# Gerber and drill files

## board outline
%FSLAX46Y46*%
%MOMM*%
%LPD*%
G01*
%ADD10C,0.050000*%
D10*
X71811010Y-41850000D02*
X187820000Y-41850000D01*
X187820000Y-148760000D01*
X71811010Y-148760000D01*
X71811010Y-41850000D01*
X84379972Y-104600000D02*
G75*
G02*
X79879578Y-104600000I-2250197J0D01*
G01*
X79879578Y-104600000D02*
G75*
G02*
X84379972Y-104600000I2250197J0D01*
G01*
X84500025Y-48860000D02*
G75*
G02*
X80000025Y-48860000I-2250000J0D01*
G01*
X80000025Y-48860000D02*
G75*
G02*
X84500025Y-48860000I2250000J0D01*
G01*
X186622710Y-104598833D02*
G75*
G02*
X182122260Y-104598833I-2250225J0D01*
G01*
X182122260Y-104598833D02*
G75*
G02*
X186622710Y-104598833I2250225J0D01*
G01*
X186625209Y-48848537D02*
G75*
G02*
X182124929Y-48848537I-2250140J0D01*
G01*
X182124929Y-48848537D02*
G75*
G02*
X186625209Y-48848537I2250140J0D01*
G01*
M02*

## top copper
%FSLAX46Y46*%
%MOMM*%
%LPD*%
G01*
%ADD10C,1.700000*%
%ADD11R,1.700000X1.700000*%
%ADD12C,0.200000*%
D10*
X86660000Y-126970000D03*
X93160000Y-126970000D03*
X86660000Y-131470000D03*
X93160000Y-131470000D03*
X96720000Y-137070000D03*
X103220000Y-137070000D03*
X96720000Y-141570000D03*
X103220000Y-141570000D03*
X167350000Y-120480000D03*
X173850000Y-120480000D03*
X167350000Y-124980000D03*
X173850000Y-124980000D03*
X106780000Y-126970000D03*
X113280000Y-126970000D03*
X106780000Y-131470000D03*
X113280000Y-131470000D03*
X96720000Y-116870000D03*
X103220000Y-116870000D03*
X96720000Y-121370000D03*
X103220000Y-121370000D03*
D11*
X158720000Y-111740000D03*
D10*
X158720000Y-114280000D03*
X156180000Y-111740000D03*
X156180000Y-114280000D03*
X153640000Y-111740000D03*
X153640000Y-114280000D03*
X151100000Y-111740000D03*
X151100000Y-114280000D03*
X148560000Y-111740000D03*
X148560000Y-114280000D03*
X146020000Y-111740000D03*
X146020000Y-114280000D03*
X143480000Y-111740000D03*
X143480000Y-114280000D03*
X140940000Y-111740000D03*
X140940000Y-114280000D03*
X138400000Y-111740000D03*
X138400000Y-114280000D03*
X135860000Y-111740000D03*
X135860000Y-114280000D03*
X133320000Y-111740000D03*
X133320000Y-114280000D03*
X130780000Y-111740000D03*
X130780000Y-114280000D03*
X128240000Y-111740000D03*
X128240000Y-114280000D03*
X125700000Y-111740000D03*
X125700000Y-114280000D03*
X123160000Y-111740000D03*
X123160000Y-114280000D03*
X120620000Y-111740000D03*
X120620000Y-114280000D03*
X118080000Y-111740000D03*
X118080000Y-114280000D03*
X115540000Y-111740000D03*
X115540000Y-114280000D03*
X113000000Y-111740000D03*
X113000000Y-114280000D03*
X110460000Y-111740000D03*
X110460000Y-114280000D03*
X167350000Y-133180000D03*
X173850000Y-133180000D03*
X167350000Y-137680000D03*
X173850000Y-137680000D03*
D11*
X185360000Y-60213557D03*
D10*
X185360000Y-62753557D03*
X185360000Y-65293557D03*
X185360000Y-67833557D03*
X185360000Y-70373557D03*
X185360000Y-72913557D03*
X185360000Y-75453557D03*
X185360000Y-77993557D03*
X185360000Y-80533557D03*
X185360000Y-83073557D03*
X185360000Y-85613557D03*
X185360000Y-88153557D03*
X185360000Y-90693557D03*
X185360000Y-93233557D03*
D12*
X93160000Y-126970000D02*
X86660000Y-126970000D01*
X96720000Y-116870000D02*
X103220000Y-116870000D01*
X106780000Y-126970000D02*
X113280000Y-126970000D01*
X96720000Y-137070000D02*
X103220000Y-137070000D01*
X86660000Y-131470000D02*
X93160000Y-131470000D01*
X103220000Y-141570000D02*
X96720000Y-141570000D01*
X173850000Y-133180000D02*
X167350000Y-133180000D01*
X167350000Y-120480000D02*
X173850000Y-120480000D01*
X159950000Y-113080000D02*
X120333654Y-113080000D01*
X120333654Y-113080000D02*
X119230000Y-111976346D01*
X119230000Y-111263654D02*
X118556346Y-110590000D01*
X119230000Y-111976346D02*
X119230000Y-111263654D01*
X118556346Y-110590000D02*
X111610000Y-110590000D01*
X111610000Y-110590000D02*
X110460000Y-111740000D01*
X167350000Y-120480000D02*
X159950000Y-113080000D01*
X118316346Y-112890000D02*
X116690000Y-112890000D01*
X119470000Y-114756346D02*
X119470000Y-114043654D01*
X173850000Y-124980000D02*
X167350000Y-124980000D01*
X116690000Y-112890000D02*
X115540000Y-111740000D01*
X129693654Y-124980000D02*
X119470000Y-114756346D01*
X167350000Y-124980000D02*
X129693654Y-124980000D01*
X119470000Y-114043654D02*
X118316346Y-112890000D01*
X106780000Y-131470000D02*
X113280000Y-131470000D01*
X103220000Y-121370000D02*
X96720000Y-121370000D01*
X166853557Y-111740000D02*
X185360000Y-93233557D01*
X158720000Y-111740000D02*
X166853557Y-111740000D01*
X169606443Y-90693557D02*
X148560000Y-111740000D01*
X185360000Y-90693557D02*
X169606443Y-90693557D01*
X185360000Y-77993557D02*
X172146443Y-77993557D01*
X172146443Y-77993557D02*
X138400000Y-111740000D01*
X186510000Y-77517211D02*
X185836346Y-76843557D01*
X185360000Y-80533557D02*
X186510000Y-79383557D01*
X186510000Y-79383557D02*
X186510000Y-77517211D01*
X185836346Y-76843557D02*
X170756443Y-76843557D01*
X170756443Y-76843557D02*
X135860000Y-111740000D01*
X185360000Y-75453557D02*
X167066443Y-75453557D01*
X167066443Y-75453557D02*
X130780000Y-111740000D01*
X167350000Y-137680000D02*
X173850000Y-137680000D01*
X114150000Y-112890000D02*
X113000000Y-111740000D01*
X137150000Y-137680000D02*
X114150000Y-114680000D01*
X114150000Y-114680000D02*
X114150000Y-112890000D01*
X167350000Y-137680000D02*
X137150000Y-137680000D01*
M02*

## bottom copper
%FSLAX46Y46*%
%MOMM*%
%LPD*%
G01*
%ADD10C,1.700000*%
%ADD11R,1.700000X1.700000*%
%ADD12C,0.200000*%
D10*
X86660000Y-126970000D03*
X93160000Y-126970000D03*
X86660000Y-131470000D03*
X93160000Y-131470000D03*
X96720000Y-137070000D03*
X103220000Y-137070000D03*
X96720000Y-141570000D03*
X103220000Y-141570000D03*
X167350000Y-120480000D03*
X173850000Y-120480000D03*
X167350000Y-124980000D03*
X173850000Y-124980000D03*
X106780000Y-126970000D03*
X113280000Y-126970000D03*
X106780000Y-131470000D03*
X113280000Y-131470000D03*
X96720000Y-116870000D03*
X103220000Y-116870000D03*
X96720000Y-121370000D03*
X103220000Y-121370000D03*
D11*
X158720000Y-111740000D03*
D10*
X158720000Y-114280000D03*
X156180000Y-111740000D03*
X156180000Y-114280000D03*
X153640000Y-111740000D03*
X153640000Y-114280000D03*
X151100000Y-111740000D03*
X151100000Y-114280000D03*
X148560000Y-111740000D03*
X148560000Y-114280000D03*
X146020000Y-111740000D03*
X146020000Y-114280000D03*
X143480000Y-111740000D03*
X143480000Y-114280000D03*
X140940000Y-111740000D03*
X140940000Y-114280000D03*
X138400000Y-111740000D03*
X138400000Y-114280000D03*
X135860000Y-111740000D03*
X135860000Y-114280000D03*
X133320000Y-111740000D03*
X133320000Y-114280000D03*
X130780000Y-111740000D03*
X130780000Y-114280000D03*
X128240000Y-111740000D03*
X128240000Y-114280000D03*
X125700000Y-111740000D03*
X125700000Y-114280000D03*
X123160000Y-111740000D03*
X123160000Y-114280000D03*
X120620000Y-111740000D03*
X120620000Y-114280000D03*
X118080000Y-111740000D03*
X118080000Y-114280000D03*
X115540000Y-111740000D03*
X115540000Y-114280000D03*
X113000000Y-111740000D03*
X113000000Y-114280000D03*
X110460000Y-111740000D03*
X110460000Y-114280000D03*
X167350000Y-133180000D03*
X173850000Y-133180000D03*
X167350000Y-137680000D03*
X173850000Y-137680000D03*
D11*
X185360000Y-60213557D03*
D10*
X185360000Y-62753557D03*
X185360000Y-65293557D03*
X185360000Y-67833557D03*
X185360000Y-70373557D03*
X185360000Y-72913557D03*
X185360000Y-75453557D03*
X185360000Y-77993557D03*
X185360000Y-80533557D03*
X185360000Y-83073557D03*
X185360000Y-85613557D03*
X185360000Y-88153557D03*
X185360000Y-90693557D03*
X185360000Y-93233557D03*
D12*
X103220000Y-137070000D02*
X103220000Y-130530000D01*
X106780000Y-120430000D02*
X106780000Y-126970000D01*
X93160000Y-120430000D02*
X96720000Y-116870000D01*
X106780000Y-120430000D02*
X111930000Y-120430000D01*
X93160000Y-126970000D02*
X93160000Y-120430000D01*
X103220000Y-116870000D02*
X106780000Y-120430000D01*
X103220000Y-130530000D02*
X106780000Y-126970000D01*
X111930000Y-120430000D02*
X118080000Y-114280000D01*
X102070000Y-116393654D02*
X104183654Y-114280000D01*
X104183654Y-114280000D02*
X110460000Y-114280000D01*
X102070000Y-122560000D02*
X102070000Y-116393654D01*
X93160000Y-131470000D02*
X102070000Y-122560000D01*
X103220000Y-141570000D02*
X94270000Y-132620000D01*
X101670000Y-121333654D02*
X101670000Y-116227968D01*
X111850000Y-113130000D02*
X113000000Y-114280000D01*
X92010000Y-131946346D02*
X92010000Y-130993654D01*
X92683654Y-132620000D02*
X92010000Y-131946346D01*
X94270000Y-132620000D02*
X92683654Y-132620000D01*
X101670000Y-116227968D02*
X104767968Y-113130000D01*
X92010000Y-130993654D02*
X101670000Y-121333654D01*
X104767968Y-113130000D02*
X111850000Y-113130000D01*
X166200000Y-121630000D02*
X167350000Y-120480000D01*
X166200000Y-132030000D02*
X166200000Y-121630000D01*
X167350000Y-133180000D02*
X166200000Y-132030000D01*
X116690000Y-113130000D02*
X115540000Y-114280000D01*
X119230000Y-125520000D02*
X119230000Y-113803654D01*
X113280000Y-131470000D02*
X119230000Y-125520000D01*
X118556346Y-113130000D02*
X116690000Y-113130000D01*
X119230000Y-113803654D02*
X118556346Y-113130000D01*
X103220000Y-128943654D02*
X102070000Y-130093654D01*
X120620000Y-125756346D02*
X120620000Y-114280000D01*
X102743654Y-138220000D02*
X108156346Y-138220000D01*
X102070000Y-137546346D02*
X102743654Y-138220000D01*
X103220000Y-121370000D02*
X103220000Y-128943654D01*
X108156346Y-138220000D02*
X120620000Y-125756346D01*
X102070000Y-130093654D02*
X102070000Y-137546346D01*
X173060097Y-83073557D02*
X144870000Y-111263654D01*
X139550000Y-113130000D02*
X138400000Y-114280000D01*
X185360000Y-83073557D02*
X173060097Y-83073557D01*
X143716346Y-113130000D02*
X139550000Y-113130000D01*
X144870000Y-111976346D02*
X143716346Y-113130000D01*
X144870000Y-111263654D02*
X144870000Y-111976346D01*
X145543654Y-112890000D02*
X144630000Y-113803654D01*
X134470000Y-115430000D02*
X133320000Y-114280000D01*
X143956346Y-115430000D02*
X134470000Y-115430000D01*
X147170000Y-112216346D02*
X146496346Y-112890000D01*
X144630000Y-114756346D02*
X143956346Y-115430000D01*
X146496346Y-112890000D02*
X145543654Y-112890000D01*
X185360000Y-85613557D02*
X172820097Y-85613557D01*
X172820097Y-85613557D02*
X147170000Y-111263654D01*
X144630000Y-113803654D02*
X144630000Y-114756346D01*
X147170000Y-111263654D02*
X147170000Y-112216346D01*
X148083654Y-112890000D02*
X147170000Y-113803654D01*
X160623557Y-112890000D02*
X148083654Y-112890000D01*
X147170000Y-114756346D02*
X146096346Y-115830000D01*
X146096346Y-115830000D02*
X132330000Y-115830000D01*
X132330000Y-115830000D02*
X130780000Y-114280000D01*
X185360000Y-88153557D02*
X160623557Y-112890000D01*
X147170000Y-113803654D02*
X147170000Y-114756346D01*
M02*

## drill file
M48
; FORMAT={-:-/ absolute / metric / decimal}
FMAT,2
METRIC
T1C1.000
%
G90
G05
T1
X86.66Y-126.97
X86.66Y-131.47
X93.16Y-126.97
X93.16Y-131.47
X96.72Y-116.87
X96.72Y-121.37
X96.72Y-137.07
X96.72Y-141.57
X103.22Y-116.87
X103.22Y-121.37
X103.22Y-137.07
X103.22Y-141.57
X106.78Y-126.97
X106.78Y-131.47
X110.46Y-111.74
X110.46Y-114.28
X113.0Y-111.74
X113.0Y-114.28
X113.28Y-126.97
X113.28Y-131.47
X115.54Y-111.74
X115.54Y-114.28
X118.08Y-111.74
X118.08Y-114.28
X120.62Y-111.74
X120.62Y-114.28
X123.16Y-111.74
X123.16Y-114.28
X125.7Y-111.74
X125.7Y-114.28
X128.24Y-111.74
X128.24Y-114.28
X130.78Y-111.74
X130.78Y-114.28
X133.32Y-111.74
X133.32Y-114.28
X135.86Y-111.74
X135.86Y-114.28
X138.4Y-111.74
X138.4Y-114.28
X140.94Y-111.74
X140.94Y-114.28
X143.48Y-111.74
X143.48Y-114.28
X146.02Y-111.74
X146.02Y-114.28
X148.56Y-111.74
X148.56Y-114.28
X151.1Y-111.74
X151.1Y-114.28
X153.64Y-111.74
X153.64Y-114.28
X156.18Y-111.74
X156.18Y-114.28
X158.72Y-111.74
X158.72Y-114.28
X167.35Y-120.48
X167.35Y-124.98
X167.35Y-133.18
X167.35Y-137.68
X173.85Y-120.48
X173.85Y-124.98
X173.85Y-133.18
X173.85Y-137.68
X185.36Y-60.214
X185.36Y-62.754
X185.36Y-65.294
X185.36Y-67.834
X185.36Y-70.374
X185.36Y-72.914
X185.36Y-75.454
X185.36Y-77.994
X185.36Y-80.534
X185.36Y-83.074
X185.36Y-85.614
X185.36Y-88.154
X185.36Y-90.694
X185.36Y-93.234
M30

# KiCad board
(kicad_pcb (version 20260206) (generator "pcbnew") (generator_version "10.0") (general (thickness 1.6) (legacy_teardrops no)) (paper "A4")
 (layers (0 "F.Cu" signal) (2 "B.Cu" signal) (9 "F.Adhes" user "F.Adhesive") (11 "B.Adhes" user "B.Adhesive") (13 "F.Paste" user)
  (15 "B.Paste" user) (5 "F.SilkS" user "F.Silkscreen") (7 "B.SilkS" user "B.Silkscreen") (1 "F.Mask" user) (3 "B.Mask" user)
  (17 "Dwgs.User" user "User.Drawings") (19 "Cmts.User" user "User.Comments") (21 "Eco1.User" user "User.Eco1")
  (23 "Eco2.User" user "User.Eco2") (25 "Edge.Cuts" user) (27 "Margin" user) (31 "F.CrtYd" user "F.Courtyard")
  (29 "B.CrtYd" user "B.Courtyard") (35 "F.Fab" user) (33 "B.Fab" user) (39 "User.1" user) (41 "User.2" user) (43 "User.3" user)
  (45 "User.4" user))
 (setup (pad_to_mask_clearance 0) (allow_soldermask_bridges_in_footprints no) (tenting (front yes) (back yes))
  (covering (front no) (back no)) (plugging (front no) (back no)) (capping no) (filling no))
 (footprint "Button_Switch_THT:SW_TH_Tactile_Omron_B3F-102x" (layer "F.Cu") (at 86.66 126.97)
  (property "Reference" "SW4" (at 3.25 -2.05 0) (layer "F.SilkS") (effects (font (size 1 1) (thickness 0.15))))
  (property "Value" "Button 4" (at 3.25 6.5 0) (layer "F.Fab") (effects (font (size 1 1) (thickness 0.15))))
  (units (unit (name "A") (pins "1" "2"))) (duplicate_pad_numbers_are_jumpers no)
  (pad "1" thru_hole circle (at 0 0) (size 1.7 1.7) (drill 1) (layers "*.Cu" "*.Mask") (remove_unused_layers no) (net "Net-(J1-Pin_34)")
   (thermal_bridge_angle 90))
  (pad "1" thru_hole circle (at 6.5 0) (size 1.7 1.7) (drill 1) (layers "*.Cu" "*.Mask") (remove_unused_layers no) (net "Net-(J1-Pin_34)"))
  (pad "2" thru_hole circle (at 0 4.5) (size 1.7 1.7) (drill 1) (layers "*.Cu" "*.Mask") (remove_unused_layers no) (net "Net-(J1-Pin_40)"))
  (pad "2" thru_hole circle (at 6.5 4.5) (size 1.7 1.7) (drill 1) (layers "*.Cu" "*.Mask") (remove_unused_layers no) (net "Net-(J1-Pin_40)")))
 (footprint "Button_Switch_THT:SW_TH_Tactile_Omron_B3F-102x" (layer "F.Cu") (at 96.72 137.07)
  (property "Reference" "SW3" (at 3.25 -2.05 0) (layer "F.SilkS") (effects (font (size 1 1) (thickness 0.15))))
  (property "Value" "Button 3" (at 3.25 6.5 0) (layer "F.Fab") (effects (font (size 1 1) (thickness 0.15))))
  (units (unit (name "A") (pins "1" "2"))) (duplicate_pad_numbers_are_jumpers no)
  (pad "1" thru_hole circle (at 0 0) (size 1.7 1.7) (drill 1) (layers "*.Cu" "*.Mask") (remove_unused_layers no) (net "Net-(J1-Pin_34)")
   (thermal_bridge_angle 90))
  (pad "1" thru_hole circle (at 6.5 0) (size 1.7 1.7) (drill 1) (layers "*.Cu" "*.Mask") (remove_unused_layers no) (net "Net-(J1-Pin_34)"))
  (pad "2" thru_hole circle (at 0 4.5) (size 1.7 1.7) (drill 1) (layers "*.Cu" "*.Mask") (remove_unused_layers no) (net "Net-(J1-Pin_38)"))
  (pad "2" thru_hole circle (at 6.5 4.5) (size 1.7 1.7) (drill 1) (layers "*.Cu" "*.Mask") (remove_unused_layers no) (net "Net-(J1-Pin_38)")))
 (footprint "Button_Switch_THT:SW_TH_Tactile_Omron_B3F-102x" (layer "F.Cu") (at 167.35 120.48)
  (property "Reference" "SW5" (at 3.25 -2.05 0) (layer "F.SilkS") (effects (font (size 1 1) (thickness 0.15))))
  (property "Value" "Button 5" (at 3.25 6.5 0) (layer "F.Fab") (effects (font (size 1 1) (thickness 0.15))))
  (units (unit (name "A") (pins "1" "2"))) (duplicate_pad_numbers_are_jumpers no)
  (pad "1" thru_hole circle (at 0 0) (size 1.7 1.7) (drill 1) (layers "*.Cu" "*.Mask") (remove_unused_layers no) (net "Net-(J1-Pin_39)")
   (thermal_bridge_angle 90))
  (pad "1" thru_hole circle (at 6.5 0) (size 1.7 1.7) (drill 1) (layers "*.Cu" "*.Mask") (remove_unused_layers no) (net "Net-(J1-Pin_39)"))
  (pad "2" thru_hole circle (at 0 4.5) (size 1.7 1.7) (drill 1) (layers "*.Cu" "*.Mask") (remove_unused_layers no) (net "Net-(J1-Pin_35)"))
  (pad "2" thru_hole circle (at 6.5 4.5) (size 1.7 1.7) (drill 1) (layers "*.Cu" "*.Mask") (remove_unused_layers no) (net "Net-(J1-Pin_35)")))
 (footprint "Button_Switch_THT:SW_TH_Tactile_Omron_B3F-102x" (layer "F.Cu") (at 106.78 126.97)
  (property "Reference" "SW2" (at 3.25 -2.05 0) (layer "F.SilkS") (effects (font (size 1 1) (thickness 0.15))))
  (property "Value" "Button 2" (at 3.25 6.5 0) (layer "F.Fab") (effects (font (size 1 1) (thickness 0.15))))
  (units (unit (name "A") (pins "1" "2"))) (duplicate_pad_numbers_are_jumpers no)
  (pad "1" thru_hole circle (at 0 0) (size 1.7 1.7) (drill 1) (layers "*.Cu" "*.Mask") (remove_unused_layers no) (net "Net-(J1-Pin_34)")
   (thermal_bridge_angle 90))
  (pad "1" thru_hole circle (at 6.5 0) (size 1.7 1.7) (drill 1) (layers "*.Cu" "*.Mask") (remove_unused_layers no) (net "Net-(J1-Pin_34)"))
  (pad "2" thru_hole circle (at 0 4.5) (size 1.7 1.7) (drill 1) (layers "*.Cu" "*.Mask") (remove_unused_layers no) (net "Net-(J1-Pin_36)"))
  (pad "2" thru_hole circle (at 6.5 4.5) (size 1.7 1.7) (drill 1) (layers "*.Cu" "*.Mask") (remove_unused_layers no) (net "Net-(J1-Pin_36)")))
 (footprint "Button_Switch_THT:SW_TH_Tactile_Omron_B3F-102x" (layer "F.Cu") (at 96.72 116.87)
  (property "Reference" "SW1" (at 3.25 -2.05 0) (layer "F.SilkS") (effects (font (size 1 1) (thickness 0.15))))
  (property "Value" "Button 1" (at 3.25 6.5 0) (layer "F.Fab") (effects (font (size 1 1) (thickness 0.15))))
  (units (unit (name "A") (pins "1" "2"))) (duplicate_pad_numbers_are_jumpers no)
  (pad "1" thru_hole circle (at 0 0) (size 1.7 1.7) (drill 1) (layers "*.Cu" "*.Mask") (remove_unused_layers no) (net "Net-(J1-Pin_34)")
   (thermal_bridge_angle 90))
  (pad "1" thru_hole circle (at 6.5 0) (size 1.7 1.7) (drill 1) (layers "*.Cu" "*.Mask") (remove_unused_layers no) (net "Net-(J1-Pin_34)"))
  (pad "2" thru_hole circle (at 0 4.5) (size 1.7 1.7) (drill 1) (layers "*.Cu" "*.Mask") (remove_unused_layers no) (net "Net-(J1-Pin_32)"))
  (pad "2" thru_hole circle (at 6.5 4.5) (size 1.7 1.7) (drill 1) (layers "*.Cu" "*.Mask") (remove_unused_layers no) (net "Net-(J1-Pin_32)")))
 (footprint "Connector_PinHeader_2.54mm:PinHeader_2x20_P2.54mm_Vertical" (layer "F.Cu") (at 158.72 111.74 -90)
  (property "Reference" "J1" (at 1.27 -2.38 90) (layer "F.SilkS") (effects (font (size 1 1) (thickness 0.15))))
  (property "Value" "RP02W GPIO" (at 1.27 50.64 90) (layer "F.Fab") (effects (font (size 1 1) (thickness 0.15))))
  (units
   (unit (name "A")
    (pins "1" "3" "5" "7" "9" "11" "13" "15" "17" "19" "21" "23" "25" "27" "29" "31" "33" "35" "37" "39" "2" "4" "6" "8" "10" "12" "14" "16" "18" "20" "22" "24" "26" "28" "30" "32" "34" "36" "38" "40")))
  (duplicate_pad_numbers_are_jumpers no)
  (pad "1" thru_hole rect (at 0 0 270) (size 1.7 1.7) (drill 1) (layers "*.Cu" "*.Mask") (remove_unused_layers no) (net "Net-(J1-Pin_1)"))
  (pad "2" thru_hole circle (at 2.54 0 270) (size 1.7 1.7) (drill 1) (layers "*.Cu" "*.Mask") (remove_unused_layers no)
   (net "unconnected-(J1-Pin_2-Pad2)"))
  (pad "3" thru_hole circle (at 0 2.54 270) (size 1.7 1.7) (drill 1) (layers "*.Cu" "*.Mask") (remove_unused_layers no)
   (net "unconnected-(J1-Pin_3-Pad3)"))
  (pad "4" thru_hole circle (at 2.54 2.54 270) (size 1.7 1.7) (drill 1) (layers "*.Cu" "*.Mask") (remove_unused_layers no)
   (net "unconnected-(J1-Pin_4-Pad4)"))
  (pad "5" thru_hole circle (at 0 5.08 270) (size 1.7 1.7) (drill 1) (layers "*.Cu" "*.Mask") (remove_unused_layers no)
   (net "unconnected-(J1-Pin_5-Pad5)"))
  (pad "6" thru_hole circle (at 2.54 5.08 270) (size 1.7 1.7) (drill 1) (layers "*.Cu" "*.Mask") (remove_unused_layers no)
   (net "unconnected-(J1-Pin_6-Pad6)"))
  (pad "7" thru_hole circle (at 0 7.62 270) (size 1.7 1.7) (drill 1) (layers "*.Cu" "*.Mask") (remove_unused_layers no)
   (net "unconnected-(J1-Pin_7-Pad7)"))
  (pad "8" thru_hole circle (at 2.54 7.62 270) (size 1.7 1.7) (drill 1) (layers "*.Cu" "*.Mask") (remove_unused_layers no)
   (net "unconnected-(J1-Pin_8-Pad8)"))
  (pad "9" thru_hole circle (at 0 10.16 270) (size 1.7 1.7) (drill 1) (layers "*.Cu" "*.Mask") (remove_unused_layers no)
   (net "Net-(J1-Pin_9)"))
  (pad "10" thru_hole circle (at 2.54 10.16 270) (size 1.7 1.7) (drill 1) (layers "*.Cu" "*.Mask") (remove_unused_layers no)
   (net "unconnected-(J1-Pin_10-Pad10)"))
  (pad "11" thru_hole circle (at 0 12.7 270) (size 1.7 1.7) (drill 1) (layers "*.Cu" "*.Mask") (remove_unused_layers no)
   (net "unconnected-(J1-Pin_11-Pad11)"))
  (pad "12" thru_hole circle (at 2.54 12.7 270) (size 1.7 1.7) (drill 1) (layers "*.Cu" "*.Mask") (remove_unused_layers no)
   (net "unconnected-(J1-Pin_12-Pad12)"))
  (pad "13" thru_hole circle (at 0 15.24 270) (size 1.7 1.7) (drill 1) (layers "*.Cu" "*.Mask") (remove_unused_layers no)
   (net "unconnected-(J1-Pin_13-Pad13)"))
  (pad "14" thru_hole circle (at 2.54 15.24 270) (size 1.7 1.7) (drill 1) (layers "*.Cu" "*.Mask") (remove_unused_layers no)
   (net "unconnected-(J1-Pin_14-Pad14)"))
  (pad "15" thru_hole circle (at 0 17.78 270) (size 1.7 1.7) (drill 1) (layers "*.Cu" "*.Mask") (remove_unused_layers no)
   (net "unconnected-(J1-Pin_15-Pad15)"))
  (pad "16" thru_hole circle (at 2.54 17.78 270) (size 1.7 1.7) (drill 1) (layers "*.Cu" "*.Mask") (remove_unused_layers no)
   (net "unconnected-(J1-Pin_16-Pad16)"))
  (pad "17" thru_hole circle (at 0 20.32 270) (size 1.7 1.7) (drill 1) (layers "*.Cu" "*.Mask") (remove_unused_layers no)
   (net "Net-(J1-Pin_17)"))
  (pad "18" thru_hole circle (at 2.54 20.32 270) (size 1.7 1.7) (drill 1) (layers "*.Cu" "*.Mask") (remove_unused_layers no)
   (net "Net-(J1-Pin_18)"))
  (pad "19" thru_hole circle (at 0 22.86 270) (size 1.7 1.7) (drill 1) (layers "*.Cu" "*.Mask") (remove_unused_layers no)
   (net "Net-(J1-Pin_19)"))
  (pad "20" thru_hole circle (at 2.54 22.86 270) (size 1.7 1.7) (drill 1) (layers "*.Cu" "*.Mask") (remove_unused_layers no)
   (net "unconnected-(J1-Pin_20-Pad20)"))
  (pad "21" thru_hole circle (at 0 25.4 270) (size 1.7 1.7) (drill 1) (layers "*.Cu" "*.Mask") (remove_unused_layers no)
   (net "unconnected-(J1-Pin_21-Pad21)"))
  (pad "22" thru_hole circle (at 2.54 25.4 270) (size 1.7 1.7) (drill 1) (layers "*.Cu" "*.Mask") (remove_unused_layers no)
   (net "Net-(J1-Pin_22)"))
  (pad "23" thru_hole circle (at 0 27.94 270) (size 1.7 1.7) (drill 1) (layers "*.Cu" "*.Mask") (remove_unused_layers no)
   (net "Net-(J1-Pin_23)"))
  (pad "24" thru_hole circle (at 2.54 27.94 270) (size 1.7 1.7) (drill 1) (layers "*.Cu" "*.Mask") (remove_unused_layers no)
   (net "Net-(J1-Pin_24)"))
  (pad "25" thru_hole circle (at 0 30.48 270) (size 1.7 1.7) (drill 1) (layers "*.Cu" "*.Mask") (remove_unused_layers no)
   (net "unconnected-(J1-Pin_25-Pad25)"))
  (pad "26" thru_hole circle (at 2.54 30.48 270) (size 1.7 1.7) (drill 1) (layers "*.Cu" "*.Mask") (remove_unused_layers no)
   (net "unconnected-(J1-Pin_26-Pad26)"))
  (pad "27" thru_hole circle (at 0 33.02 270) (size 1.7 1.7) (drill 1) (layers "*.Cu" "*.Mask") (remove_unused_layers no)
   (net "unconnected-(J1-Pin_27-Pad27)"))
  (pad "28" thru_hole circle (at 2.54 33.02 270) (size 1.7 1.7) (drill 1) (layers "*.Cu" "*.Mask") (remove_unused_layers no)
   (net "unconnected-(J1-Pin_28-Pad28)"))
  (pad "29" thru_hole circle (at 0 35.56 270) (size 1.7 1.7) (drill 1) (layers "*.Cu" "*.Mask") (remove_unused_layers no)
   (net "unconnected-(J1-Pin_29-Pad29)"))
  (pad "30" thru_hole circle (at 2.54 35.56 270) (size 1.7 1.7) (drill 1) (layers "*.Cu" "*.Mask") (remove_unused_layers no)
   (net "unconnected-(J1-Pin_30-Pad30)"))
  (pad "31" thru_hole circle (at 0 38.1 270) (size 1.7 1.7) (drill 1) (layers "*.Cu" "*.Mask") (remove_unused_layers no)
   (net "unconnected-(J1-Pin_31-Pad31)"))
  (pad "32" thru_hole circle (at 2.54 38.1 270) (size 1.7 1.7) (drill 1) (layers "*.Cu" "*.Mask") (remove_unused_layers no)
   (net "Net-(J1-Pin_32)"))
  (pad "33" thru_hole circle (at 0 40.64 270) (size 1.7 1.7) (drill 1) (layers "*.Cu" "*.Mask") (remove_unused_layers no)
   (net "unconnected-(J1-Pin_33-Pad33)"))
  (pad "34" thru_hole circle (at 2.54 40.64 270) (size 1.7 1.7) (drill 1) (layers "*.Cu" "*.Mask") (remove_unused_layers no)
   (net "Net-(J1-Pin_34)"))
  (pad "35" thru_hole circle (at 0 43.18 270) (size 1.7 1.7) (drill 1) (layers "*.Cu" "*.Mask") (remove_unused_layers no)
   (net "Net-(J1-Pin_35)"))
  (pad "36" thru_hole circle (at 2.54 43.18 270) (size 1.7 1.7) (drill 1) (layers "*.Cu" "*.Mask") (remove_unused_layers no)
   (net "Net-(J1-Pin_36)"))
  (pad "37" thru_hole circle (at 0 45.72 270) (size 1.7 1.7) (drill 1) (layers "*.Cu" "*.Mask") (remove_unused_layers no)
   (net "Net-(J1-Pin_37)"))
  (pad "38" thru_hole circle (at 2.54 45.72 270) (size 1.7 1.7) (drill 1) (layers "*.Cu" "*.Mask") (remove_unused_layers no)
   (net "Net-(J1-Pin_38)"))
  (pad "39" thru_hole circle (at 0 48.26 270) (size 1.7 1.7) (drill 1) (layers "*.Cu" "*.Mask") (remove_unused_layers no)
   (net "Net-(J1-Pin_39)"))
  (pad "40" thru_hole circle (at 2.54 48.26 270) (size 1.7 1.7) (drill 1) (layers "*.Cu" "*.Mask") (remove_unused_layers no)
   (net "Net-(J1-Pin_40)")))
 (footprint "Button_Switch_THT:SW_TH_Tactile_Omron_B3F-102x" (layer "F.Cu") (at 167.35 133.18)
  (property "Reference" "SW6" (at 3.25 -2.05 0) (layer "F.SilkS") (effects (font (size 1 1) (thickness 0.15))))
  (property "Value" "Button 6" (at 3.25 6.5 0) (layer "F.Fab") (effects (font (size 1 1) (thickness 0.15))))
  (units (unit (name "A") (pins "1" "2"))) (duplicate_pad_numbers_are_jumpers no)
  (pad "1" thru_hole circle (at 0 0) (size 1.7 1.7) (drill 1) (layers "*.Cu" "*.Mask") (remove_unused_layers no) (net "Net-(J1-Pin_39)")
   (thermal_bridge_angle 90))
  (pad "1" thru_hole circle (at 6.5 0) (size 1.7 1.7) (drill 1) (layers "*.Cu" "*.Mask") (remove_unused_layers no) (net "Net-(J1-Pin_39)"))
  (pad "2" thru_hole circle (at 0 4.5) (size 1.7 1.7) (drill 1) (layers "*.Cu" "*.Mask") (remove_unused_layers no) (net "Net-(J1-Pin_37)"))
  (pad "2" thru_hole circle (at 6.5 4.5) (size 1.7 1.7) (drill 1) (layers "*.Cu" "*.Mask") (remove_unused_layers no) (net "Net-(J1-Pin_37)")))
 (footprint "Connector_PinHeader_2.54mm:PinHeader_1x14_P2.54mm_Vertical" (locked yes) (layer "F.Cu") (at 185.36 60.213557)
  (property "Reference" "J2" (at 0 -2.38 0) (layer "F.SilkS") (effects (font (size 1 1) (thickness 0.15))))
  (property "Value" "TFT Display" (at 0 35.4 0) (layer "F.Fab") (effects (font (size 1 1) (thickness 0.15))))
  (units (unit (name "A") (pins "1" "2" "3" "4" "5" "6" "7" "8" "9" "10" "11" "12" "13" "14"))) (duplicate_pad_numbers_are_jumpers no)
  (pad "1" thru_hole rect (at 0 0) (size 1.7 1.7) (drill 1) (layers "*.Cu" "*.Mask") (remove_unused_layers no)
   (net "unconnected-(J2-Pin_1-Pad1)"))
  (pad "2" thru_hole circle (at 0 2.54) (size 1.7 1.7) (drill 1) (layers "*.Cu" "*.Mask") (remove_unused_layers no)
   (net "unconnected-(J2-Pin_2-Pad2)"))
  (pad "3" thru_hole circle (at 0 5.08) (size 1.7 1.7) (drill 1) (layers "*.Cu" "*.Mask") (remove_unused_layers no)
   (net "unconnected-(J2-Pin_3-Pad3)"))
  (pad "4" thru_hole circle (at 0 7.62) (size 1.7 1.7) (drill 1) (layers "*.Cu" "*.Mask") (remove_unused_layers no)
   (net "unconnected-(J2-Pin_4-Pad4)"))
  (pad "5" thru_hole circle (at 0 10.16) (size 1.7 1.7) (drill 1) (layers "*.Cu" "*.Mask") (remove_unused_layers no)
   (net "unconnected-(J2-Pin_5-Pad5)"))
  (pad "6" thru_hole circle (at 0 12.7) (size 1.7 1.7) (drill 1) (layers "*.Cu" "*.Mask") (remove_unused_layers no)
   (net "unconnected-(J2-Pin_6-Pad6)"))
  (pad "7" thru_hole circle (at 0 15.24) (size 1.7 1.7) (drill 1) (layers "*.Cu" "*.Mask") (remove_unused_layers no) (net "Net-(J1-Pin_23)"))
  (pad "8" thru_hole circle (at 0 17.78) (size 1.7 1.7) (drill 1) (layers "*.Cu" "*.Mask") (remove_unused_layers no) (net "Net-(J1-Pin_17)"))
  (pad "9" thru_hole circle (at 0 20.32) (size 1.7 1.7) (drill 1) (layers "*.Cu" "*.Mask") (remove_unused_layers no) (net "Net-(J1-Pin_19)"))
  (pad "10" thru_hole circle (at 0 22.86) (size 1.7 1.7) (drill 1) (layers "*.Cu" "*.Mask") (remove_unused_layers no)
   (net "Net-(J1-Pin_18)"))
  (pad "11" thru_hole circle (at 0 25.4) (size 1.7 1.7) (drill 1) (layers "*.Cu" "*.Mask") (remove_unused_layers no) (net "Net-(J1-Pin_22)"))
  (pad "12" thru_hole circle (at 0 27.94) (size 1.7 1.7) (drill 1) (layers "*.Cu" "*.Mask") (remove_unused_layers no)
   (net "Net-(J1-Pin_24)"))
  (pad "13" thru_hole circle (at 0 30.48) (size 1.7 1.7) (drill 1) (layers "*.Cu" "*.Mask") (remove_unused_layers no) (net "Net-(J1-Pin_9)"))
  (pad "14" thru_hole circle (at 0 33.02) (size 1.7 1.7) (drill 1) (layers "*.Cu" "*.Mask") (remove_unused_layers no) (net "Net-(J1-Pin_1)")))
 (gr_rect (start 71.81101 41.85) (end 187.82 148.76) (stroke (width 0.05) (type default)) (fill no) (layer "Edge.Cuts"))
 (gr_circle (center 82.129775 104.6) (end 82.1 106.85) (stroke (width 0.05) (type default)) (fill no) (locked yes) (layer "Edge.Cuts"))
 (gr_circle (center 82.250025 48.86) (end 82.25 46.61) (stroke (width 0.05) (type default)) (fill no) (locked yes) (layer "Edge.Cuts"))
 (gr_circle (center 184.372485 104.598833) (end 186.61 104.36) (stroke (width 0.05) (type default)) (fill no) (locked yes)
  (layer "Edge.Cuts"))
 (gr_circle (center 184.375069 48.848537) (end 184.46 46.6) (stroke (width 0.05) (type default)) (fill no) (locked yes) (layer "Edge.Cuts"))
 (segment (start 93.16 126.97) (end 86.66 126.97) (width 0.2) (layer "F.Cu") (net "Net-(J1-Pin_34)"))
 (segment (start 96.72 116.87) (end 103.22 116.87) (width 0.2) (layer "F.Cu") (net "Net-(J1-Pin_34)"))
 (segment (start 106.78 126.97) (end 113.28 126.97) (width 0.2) (layer "F.Cu") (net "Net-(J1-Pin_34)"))
 (segment (start 96.72 137.07) (end 103.22 137.07) (width 0.2) (layer "F.Cu") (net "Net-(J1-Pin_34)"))
 (segment (start 103.22 137.07) (end 103.22 130.53) (width 0.2) (layer "B.Cu") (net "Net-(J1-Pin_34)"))
 (segment (start 106.78 120.43) (end 106.78 126.97) (width 0.2) (layer "B.Cu") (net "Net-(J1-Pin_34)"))
 (segment (start 93.16 120.43) (end 96.72 116.87) (width 0.2) (layer "B.Cu") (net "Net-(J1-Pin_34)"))
 (segment (start 106.78 120.43) (end 111.93 120.43) (width 0.2) (layer "B.Cu") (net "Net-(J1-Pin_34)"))
 (segment (start 93.16 126.97) (end 93.16 120.43) (width 0.2) (layer "B.Cu") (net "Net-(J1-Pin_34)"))
 (segment (start 103.22 116.87) (end 106.78 120.43) (width 0.2) (layer "B.Cu") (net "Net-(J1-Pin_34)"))
 (segment (start 103.22 130.53) (end 106.78 126.97) (width 0.2) (layer "B.Cu") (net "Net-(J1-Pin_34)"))
 (segment (start 111.93 120.43) (end 118.08 114.28) (width 0.2) (layer "B.Cu") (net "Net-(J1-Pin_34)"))
 (segment (start 86.66 131.47) (end 93.16 131.47) (width 0.2) (layer "F.Cu") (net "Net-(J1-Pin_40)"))
 (segment (start 102.07 116.393654) (end 104.183654 114.28) (width 0.2) (layer "B.Cu") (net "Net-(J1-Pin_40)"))
 (segment (start 104.183654 114.28) (end 110.46 114.28) (width 0.2) (layer "B.Cu") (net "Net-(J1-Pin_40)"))
 (segment (start 102.07 122.56) (end 102.07 116.393654) (width 0.2) (layer "B.Cu") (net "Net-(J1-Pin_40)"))
 (segment (start 93.16 131.47) (end 102.07 122.56) (width 0.2) (layer "B.Cu") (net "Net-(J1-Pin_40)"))
 (segment (start 103.22 141.57) (end 96.72 141.57) (width 0.2) (layer "F.Cu") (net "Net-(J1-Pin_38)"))
 (segment (start 103.22 141.57) (end 94.27 132.62) (width 0.2) (layer "B.Cu") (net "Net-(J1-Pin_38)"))
 (segment (start 101.67 121.333654) (end 101.67 116.227968) (width 0.2) (layer "B.Cu") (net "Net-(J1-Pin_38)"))
 (segment (start 111.85 113.13) (end 113 114.28) (width 0.2) (layer "B.Cu") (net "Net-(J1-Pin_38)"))
 (segment (start 92.01 131.946346) (end 92.01 130.993654) (width 0.2) (layer "B.Cu") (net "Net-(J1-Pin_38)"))
 (segment (start 92.683654 132.62) (end 92.01 131.946346) (width 0.2) (layer "B.Cu") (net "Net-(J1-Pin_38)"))
 (segment (start 94.27 132.62) (end 92.683654 132.62) (width 0.2) (layer "B.Cu") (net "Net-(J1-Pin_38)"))
 (segment (start 101.67 116.227968) (end 104.767968 113.13) (width 0.2) (layer "B.Cu") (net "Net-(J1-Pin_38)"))
 (segment (start 92.01 130.993654) (end 101.67 121.333654) (width 0.2) (layer "B.Cu") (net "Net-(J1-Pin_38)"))
 (segment (start 104.767968 113.13) (end 111.85 113.13) (width 0.2) (layer "B.Cu") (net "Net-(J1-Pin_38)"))
 (segment (start 173.85 133.18) (end 167.35 133.18) (width 0.2) (layer "F.Cu") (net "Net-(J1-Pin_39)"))
 (segment (start 167.35 120.48) (end 173.85 120.48) (width 0.2) (layer "F.Cu") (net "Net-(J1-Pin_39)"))
 (segment (start 159.95 113.08) (end 120.333654 113.08) (width 0.2) (layer "F.Cu") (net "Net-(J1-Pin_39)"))
 (segment (start 120.333654 113.08) (end 119.23 111.976346) (width 0.2) (layer "F.Cu") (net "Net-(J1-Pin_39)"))
 (segment (start 119.23 111.263654) (end 118.556346 110.59) (width 0.2) (layer "F.Cu") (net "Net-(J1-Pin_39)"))
 (segment (start 119.23 111.976346) (end 119.23 111.263654) (width 0.2) (layer "F.Cu") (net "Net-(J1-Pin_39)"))
 (segment (start 118.556346 110.59) (end 111.61 110.59) (width 0.2) (layer "F.Cu") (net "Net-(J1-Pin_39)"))
 (segment (start 111.61 110.59) (end 110.46 111.74) (width 0.2) (layer "F.Cu") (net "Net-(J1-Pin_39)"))
 (segment (start 167.35 120.48) (end 159.95 113.08) (width 0.2) (layer "F.Cu") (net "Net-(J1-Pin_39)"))
 (segment (start 166.2 121.63) (end 167.35 120.48) (width 0.2) (layer "B.Cu") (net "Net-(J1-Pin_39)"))
 (segment (start 166.2 132.03) (end 166.2 121.63) (width 0.2) (layer "B.Cu") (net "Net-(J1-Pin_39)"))
 (segment (start 167.35 133.18) (end 166.2 132.03) (width 0.2) (layer "B.Cu") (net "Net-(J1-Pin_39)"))
 (segment (start 118.316346 112.89) (end 116.69 112.89) (width 0.2) (layer "F.Cu") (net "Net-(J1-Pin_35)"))
 (segment (start 119.47 114.756346) (end 119.47 114.043654) (width 0.2) (layer "F.Cu") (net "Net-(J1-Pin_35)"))
 (segment (start 173.85 124.98) (end 167.35 124.98) (width 0.2) (layer "F.Cu") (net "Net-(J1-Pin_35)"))
 (segment (start 116.69 112.89) (end 115.54 111.74) (width 0.2) (layer "F.Cu") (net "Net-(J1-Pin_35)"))
 (segment (start 129.693654 124.98) (end 119.47 114.756346) (width 0.2) (layer "F.Cu") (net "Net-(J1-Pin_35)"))
 (segment (start 167.35 124.98) (end 129.693654 124.98) (width 0.2) (layer "F.Cu") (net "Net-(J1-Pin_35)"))
 (segment (start 119.47 114.043654) (end 118.316346 112.89) (width 0.2) (layer "F.Cu") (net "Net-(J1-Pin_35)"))
 (segment (start 106.78 131.47) (end 113.28 131.47) (width 0.2) (layer "F.Cu") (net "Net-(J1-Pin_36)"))
 (segment (start 116.69 113.13) (end 115.54 114.28) (width 0.2) (layer "B.Cu") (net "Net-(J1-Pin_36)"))
 (segment (start 119.23 125.52) (end 119.23 113.803654) (width 0.2) (layer "B.Cu") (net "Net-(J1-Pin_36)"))
 (segment (start 113.28 131.47) (end 119.23 125.52) (width 0.2) (layer "B.Cu") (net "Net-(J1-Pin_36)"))
 (segment (start 118.556346 113.13) (end 116.69 113.13) (width 0.2) (layer "B.Cu") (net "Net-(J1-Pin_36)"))
 (segment (start 119.23 113.803654) (end 118.556346 113.13) (width 0.2) (layer "B.Cu") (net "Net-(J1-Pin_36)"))
 (segment (start 103.22 121.37) (end 96.72 121.37) (width 0.2) (layer "F.Cu") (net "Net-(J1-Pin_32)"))
 (segment (start 103.22 128.943654) (end 102.07 130.093654) (width 0.2) (layer "B.Cu") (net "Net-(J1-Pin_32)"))
 (segment (start 120.62 125.756346) (end 120.62 114.28) (width 0.2) (layer "B.Cu") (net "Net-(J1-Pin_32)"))
 (segment (start 102.743654 138.22) (end 108.156346 138.22) (width 0.2) (layer "B.Cu") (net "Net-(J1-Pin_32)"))
 (segment (start 102.07 137.546346) (end 102.743654 138.22) (width 0.2) (layer "B.Cu") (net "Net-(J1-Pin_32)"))
 (segment (start 103.22 121.37) (end 103.22 128.943654) (width 0.2) (layer "B.Cu") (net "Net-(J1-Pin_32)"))
 (segment (start 108.156346 138.22) (end 120.62 125.756346) (width 0.2) (layer "B.Cu") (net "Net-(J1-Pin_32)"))
 (segment (start 102.07 130.093654) (end 102.07 137.546346) (width 0.2) (layer "B.Cu") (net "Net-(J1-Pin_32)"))
 (segment (start 166.853557 111.74) (end 185.36 93.233557) (width 0.2) (layer "F.Cu") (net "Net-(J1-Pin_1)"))
 (segment (start 158.72 111.74) (end 166.853557 111.74) (width 0.2) (layer "F.Cu") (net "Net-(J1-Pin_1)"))
 (segment (start 169.606443 90.693557) (end 148.56 111.74) (width 0.2) (layer "F.Cu") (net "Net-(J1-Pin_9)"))
 (segment (start 185.36 90.693557) (end 169.606443 90.693557) (width 0.2) (layer "F.Cu") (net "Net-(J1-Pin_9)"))
 (segment (start 185.36 77.993557) (end 172.146443 77.993557) (width 0.2) (layer "F.Cu") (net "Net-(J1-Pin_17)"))
 (segment (start 172.146443 77.993557) (end 138.4 111.74) (width 0.2) (layer "F.Cu") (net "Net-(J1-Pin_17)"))
 (segment (start 173.060097 83.073557) (end 144.87 111.263654) (width 0.2) (layer "B.Cu") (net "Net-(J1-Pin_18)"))
 (segment (start 139.55 113.13) (end 138.4 114.28) (width 0.2) (layer "B.Cu") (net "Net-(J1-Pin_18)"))
 (segment (start 185.36 83.073557) (end 173.060097 83.073557) (width 0.2) (layer "B.Cu") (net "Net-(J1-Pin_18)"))
 (segment (start 143.716346 113.13) (end 139.55 113.13) (width 0.2) (layer "B.Cu") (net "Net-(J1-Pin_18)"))
 (segment (start 144.87 111.976346) (end 143.716346 113.13) (width 0.2) (layer "B.Cu") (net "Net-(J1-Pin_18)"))
 (segment (start 144.87 111.263654) (end 144.87 111.976346) (width 0.2) (layer "B.Cu") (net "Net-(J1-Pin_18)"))
 (segment (start 186.51 77.517211) (end 185.836346 76.843557) (width 0.2) (layer "F.Cu") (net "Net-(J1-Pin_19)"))
 (segment (start 185.36 80.533557) (end 186.51 79.383557) (width 0.2) (layer "F.Cu") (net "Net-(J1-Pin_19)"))
 (segment (start 186.51 79.383557) (end 186.51 77.517211) (width 0.2) (layer "F.Cu") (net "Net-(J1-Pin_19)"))
 (segment (start 185.836346 76.843557) (end 170.756443 76.843557) (width 0.2) (layer "F.Cu") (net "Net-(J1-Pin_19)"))
 (segment (start 170.756443 76.843557) (end 135.86 111.74) (width 0.2) (layer "F.Cu") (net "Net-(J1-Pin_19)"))
 (segment (start 145.543654 112.89) (end 144.63 113.803654) (width 0.2) (layer "B.Cu") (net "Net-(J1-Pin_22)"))
 (segment (start 134.47 115.43) (end 133.32 114.28) (width 0.2) (layer "B.Cu") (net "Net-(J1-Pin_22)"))
 (segment (start 143.956346 115.43) (end 134.47 115.43) (width 0.2) (layer "B.Cu") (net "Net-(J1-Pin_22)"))
 (segment (start 147.17 112.216346) (end 146.496346 112.89) (width 0.2) (layer "B.Cu") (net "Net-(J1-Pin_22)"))
 (segment (start 144.63 114.756346) (end 143.956346 115.43) (width 0.2) (layer "B.Cu") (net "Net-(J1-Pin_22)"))
 (segment (start 146.496346 112.89) (end 145.543654 112.89) (width 0.2) (layer "B.Cu") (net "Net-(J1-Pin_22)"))
 (segment (start 185.36 85.613557) (end 172.820097 85.613557) (width 0.2) (layer "B.Cu") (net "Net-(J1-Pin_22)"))
 (segment (start 172.820097 85.613557) (end 147.17 111.263654) (width 0.2) (layer "B.Cu") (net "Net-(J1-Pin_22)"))
 (segment (start 144.63 113.803654) (end 144.63 114.756346) (width 0.2) (layer "B.Cu") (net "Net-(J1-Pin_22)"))
 (segment (start 147.17 111.263654) (end 147.17 112.216346) (width 0.2) (layer "B.Cu") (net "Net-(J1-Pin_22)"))
 (segment (start 185.36 75.453557) (end 167.066443 75.453557) (width 0.2) (layer "F.Cu") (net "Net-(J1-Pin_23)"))
 (segment (start 167.066443 75.453557) (end 130.78 111.74) (width 0.2) (layer "F.Cu") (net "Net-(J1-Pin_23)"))
 (segment (start 148.083654 112.89) (end 147.17 113.803654) (width 0.2) (layer "B.Cu") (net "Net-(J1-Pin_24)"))
 (segment (start 160.623557 112.89) (end 148.083654 112.89) (width 0.2) (layer "B.Cu") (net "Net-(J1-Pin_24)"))
 (segment (start 147.17 114.756346) (end 146.096346 115.83) (width 0.2) (layer "B.Cu") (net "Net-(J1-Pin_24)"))
 (segment (start 146.096346 115.83) (end 132.33 115.83) (width 0.2) (layer "B.Cu") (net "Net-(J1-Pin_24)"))
 (segment (start 132.33 115.83) (end 130.78 114.28) (width 0.2) (layer "B.Cu") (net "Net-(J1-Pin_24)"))
 (segment (start 185.36 88.153557) (end 160.623557 112.89) (width 0.2) (layer "B.Cu") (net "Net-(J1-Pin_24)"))
 (segment (start 147.17 113.803654) (end 147.17 114.756346) (width 0.2) (layer "B.Cu") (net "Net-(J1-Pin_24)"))
 (segment (start 167.35 137.68) (end 173.85 137.68) (width 0.2) (layer "F.Cu") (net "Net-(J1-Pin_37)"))
 (segment (start 114.15 112.89) (end 113 111.74) (width 0.2) (layer "F.Cu") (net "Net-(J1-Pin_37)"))
 (segment (start 137.15 137.68) (end 114.15 114.68) (width 0.2) (layer "F.Cu") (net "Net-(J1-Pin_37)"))
 (segment (start 114.15 114.68) (end 114.15 112.89) (width 0.2) (layer "F.Cu") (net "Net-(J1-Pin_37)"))
 (segment (start 167.35 137.68) (end 137.15 137.68) (width 0.2) (layer "F.Cu") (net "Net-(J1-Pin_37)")))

